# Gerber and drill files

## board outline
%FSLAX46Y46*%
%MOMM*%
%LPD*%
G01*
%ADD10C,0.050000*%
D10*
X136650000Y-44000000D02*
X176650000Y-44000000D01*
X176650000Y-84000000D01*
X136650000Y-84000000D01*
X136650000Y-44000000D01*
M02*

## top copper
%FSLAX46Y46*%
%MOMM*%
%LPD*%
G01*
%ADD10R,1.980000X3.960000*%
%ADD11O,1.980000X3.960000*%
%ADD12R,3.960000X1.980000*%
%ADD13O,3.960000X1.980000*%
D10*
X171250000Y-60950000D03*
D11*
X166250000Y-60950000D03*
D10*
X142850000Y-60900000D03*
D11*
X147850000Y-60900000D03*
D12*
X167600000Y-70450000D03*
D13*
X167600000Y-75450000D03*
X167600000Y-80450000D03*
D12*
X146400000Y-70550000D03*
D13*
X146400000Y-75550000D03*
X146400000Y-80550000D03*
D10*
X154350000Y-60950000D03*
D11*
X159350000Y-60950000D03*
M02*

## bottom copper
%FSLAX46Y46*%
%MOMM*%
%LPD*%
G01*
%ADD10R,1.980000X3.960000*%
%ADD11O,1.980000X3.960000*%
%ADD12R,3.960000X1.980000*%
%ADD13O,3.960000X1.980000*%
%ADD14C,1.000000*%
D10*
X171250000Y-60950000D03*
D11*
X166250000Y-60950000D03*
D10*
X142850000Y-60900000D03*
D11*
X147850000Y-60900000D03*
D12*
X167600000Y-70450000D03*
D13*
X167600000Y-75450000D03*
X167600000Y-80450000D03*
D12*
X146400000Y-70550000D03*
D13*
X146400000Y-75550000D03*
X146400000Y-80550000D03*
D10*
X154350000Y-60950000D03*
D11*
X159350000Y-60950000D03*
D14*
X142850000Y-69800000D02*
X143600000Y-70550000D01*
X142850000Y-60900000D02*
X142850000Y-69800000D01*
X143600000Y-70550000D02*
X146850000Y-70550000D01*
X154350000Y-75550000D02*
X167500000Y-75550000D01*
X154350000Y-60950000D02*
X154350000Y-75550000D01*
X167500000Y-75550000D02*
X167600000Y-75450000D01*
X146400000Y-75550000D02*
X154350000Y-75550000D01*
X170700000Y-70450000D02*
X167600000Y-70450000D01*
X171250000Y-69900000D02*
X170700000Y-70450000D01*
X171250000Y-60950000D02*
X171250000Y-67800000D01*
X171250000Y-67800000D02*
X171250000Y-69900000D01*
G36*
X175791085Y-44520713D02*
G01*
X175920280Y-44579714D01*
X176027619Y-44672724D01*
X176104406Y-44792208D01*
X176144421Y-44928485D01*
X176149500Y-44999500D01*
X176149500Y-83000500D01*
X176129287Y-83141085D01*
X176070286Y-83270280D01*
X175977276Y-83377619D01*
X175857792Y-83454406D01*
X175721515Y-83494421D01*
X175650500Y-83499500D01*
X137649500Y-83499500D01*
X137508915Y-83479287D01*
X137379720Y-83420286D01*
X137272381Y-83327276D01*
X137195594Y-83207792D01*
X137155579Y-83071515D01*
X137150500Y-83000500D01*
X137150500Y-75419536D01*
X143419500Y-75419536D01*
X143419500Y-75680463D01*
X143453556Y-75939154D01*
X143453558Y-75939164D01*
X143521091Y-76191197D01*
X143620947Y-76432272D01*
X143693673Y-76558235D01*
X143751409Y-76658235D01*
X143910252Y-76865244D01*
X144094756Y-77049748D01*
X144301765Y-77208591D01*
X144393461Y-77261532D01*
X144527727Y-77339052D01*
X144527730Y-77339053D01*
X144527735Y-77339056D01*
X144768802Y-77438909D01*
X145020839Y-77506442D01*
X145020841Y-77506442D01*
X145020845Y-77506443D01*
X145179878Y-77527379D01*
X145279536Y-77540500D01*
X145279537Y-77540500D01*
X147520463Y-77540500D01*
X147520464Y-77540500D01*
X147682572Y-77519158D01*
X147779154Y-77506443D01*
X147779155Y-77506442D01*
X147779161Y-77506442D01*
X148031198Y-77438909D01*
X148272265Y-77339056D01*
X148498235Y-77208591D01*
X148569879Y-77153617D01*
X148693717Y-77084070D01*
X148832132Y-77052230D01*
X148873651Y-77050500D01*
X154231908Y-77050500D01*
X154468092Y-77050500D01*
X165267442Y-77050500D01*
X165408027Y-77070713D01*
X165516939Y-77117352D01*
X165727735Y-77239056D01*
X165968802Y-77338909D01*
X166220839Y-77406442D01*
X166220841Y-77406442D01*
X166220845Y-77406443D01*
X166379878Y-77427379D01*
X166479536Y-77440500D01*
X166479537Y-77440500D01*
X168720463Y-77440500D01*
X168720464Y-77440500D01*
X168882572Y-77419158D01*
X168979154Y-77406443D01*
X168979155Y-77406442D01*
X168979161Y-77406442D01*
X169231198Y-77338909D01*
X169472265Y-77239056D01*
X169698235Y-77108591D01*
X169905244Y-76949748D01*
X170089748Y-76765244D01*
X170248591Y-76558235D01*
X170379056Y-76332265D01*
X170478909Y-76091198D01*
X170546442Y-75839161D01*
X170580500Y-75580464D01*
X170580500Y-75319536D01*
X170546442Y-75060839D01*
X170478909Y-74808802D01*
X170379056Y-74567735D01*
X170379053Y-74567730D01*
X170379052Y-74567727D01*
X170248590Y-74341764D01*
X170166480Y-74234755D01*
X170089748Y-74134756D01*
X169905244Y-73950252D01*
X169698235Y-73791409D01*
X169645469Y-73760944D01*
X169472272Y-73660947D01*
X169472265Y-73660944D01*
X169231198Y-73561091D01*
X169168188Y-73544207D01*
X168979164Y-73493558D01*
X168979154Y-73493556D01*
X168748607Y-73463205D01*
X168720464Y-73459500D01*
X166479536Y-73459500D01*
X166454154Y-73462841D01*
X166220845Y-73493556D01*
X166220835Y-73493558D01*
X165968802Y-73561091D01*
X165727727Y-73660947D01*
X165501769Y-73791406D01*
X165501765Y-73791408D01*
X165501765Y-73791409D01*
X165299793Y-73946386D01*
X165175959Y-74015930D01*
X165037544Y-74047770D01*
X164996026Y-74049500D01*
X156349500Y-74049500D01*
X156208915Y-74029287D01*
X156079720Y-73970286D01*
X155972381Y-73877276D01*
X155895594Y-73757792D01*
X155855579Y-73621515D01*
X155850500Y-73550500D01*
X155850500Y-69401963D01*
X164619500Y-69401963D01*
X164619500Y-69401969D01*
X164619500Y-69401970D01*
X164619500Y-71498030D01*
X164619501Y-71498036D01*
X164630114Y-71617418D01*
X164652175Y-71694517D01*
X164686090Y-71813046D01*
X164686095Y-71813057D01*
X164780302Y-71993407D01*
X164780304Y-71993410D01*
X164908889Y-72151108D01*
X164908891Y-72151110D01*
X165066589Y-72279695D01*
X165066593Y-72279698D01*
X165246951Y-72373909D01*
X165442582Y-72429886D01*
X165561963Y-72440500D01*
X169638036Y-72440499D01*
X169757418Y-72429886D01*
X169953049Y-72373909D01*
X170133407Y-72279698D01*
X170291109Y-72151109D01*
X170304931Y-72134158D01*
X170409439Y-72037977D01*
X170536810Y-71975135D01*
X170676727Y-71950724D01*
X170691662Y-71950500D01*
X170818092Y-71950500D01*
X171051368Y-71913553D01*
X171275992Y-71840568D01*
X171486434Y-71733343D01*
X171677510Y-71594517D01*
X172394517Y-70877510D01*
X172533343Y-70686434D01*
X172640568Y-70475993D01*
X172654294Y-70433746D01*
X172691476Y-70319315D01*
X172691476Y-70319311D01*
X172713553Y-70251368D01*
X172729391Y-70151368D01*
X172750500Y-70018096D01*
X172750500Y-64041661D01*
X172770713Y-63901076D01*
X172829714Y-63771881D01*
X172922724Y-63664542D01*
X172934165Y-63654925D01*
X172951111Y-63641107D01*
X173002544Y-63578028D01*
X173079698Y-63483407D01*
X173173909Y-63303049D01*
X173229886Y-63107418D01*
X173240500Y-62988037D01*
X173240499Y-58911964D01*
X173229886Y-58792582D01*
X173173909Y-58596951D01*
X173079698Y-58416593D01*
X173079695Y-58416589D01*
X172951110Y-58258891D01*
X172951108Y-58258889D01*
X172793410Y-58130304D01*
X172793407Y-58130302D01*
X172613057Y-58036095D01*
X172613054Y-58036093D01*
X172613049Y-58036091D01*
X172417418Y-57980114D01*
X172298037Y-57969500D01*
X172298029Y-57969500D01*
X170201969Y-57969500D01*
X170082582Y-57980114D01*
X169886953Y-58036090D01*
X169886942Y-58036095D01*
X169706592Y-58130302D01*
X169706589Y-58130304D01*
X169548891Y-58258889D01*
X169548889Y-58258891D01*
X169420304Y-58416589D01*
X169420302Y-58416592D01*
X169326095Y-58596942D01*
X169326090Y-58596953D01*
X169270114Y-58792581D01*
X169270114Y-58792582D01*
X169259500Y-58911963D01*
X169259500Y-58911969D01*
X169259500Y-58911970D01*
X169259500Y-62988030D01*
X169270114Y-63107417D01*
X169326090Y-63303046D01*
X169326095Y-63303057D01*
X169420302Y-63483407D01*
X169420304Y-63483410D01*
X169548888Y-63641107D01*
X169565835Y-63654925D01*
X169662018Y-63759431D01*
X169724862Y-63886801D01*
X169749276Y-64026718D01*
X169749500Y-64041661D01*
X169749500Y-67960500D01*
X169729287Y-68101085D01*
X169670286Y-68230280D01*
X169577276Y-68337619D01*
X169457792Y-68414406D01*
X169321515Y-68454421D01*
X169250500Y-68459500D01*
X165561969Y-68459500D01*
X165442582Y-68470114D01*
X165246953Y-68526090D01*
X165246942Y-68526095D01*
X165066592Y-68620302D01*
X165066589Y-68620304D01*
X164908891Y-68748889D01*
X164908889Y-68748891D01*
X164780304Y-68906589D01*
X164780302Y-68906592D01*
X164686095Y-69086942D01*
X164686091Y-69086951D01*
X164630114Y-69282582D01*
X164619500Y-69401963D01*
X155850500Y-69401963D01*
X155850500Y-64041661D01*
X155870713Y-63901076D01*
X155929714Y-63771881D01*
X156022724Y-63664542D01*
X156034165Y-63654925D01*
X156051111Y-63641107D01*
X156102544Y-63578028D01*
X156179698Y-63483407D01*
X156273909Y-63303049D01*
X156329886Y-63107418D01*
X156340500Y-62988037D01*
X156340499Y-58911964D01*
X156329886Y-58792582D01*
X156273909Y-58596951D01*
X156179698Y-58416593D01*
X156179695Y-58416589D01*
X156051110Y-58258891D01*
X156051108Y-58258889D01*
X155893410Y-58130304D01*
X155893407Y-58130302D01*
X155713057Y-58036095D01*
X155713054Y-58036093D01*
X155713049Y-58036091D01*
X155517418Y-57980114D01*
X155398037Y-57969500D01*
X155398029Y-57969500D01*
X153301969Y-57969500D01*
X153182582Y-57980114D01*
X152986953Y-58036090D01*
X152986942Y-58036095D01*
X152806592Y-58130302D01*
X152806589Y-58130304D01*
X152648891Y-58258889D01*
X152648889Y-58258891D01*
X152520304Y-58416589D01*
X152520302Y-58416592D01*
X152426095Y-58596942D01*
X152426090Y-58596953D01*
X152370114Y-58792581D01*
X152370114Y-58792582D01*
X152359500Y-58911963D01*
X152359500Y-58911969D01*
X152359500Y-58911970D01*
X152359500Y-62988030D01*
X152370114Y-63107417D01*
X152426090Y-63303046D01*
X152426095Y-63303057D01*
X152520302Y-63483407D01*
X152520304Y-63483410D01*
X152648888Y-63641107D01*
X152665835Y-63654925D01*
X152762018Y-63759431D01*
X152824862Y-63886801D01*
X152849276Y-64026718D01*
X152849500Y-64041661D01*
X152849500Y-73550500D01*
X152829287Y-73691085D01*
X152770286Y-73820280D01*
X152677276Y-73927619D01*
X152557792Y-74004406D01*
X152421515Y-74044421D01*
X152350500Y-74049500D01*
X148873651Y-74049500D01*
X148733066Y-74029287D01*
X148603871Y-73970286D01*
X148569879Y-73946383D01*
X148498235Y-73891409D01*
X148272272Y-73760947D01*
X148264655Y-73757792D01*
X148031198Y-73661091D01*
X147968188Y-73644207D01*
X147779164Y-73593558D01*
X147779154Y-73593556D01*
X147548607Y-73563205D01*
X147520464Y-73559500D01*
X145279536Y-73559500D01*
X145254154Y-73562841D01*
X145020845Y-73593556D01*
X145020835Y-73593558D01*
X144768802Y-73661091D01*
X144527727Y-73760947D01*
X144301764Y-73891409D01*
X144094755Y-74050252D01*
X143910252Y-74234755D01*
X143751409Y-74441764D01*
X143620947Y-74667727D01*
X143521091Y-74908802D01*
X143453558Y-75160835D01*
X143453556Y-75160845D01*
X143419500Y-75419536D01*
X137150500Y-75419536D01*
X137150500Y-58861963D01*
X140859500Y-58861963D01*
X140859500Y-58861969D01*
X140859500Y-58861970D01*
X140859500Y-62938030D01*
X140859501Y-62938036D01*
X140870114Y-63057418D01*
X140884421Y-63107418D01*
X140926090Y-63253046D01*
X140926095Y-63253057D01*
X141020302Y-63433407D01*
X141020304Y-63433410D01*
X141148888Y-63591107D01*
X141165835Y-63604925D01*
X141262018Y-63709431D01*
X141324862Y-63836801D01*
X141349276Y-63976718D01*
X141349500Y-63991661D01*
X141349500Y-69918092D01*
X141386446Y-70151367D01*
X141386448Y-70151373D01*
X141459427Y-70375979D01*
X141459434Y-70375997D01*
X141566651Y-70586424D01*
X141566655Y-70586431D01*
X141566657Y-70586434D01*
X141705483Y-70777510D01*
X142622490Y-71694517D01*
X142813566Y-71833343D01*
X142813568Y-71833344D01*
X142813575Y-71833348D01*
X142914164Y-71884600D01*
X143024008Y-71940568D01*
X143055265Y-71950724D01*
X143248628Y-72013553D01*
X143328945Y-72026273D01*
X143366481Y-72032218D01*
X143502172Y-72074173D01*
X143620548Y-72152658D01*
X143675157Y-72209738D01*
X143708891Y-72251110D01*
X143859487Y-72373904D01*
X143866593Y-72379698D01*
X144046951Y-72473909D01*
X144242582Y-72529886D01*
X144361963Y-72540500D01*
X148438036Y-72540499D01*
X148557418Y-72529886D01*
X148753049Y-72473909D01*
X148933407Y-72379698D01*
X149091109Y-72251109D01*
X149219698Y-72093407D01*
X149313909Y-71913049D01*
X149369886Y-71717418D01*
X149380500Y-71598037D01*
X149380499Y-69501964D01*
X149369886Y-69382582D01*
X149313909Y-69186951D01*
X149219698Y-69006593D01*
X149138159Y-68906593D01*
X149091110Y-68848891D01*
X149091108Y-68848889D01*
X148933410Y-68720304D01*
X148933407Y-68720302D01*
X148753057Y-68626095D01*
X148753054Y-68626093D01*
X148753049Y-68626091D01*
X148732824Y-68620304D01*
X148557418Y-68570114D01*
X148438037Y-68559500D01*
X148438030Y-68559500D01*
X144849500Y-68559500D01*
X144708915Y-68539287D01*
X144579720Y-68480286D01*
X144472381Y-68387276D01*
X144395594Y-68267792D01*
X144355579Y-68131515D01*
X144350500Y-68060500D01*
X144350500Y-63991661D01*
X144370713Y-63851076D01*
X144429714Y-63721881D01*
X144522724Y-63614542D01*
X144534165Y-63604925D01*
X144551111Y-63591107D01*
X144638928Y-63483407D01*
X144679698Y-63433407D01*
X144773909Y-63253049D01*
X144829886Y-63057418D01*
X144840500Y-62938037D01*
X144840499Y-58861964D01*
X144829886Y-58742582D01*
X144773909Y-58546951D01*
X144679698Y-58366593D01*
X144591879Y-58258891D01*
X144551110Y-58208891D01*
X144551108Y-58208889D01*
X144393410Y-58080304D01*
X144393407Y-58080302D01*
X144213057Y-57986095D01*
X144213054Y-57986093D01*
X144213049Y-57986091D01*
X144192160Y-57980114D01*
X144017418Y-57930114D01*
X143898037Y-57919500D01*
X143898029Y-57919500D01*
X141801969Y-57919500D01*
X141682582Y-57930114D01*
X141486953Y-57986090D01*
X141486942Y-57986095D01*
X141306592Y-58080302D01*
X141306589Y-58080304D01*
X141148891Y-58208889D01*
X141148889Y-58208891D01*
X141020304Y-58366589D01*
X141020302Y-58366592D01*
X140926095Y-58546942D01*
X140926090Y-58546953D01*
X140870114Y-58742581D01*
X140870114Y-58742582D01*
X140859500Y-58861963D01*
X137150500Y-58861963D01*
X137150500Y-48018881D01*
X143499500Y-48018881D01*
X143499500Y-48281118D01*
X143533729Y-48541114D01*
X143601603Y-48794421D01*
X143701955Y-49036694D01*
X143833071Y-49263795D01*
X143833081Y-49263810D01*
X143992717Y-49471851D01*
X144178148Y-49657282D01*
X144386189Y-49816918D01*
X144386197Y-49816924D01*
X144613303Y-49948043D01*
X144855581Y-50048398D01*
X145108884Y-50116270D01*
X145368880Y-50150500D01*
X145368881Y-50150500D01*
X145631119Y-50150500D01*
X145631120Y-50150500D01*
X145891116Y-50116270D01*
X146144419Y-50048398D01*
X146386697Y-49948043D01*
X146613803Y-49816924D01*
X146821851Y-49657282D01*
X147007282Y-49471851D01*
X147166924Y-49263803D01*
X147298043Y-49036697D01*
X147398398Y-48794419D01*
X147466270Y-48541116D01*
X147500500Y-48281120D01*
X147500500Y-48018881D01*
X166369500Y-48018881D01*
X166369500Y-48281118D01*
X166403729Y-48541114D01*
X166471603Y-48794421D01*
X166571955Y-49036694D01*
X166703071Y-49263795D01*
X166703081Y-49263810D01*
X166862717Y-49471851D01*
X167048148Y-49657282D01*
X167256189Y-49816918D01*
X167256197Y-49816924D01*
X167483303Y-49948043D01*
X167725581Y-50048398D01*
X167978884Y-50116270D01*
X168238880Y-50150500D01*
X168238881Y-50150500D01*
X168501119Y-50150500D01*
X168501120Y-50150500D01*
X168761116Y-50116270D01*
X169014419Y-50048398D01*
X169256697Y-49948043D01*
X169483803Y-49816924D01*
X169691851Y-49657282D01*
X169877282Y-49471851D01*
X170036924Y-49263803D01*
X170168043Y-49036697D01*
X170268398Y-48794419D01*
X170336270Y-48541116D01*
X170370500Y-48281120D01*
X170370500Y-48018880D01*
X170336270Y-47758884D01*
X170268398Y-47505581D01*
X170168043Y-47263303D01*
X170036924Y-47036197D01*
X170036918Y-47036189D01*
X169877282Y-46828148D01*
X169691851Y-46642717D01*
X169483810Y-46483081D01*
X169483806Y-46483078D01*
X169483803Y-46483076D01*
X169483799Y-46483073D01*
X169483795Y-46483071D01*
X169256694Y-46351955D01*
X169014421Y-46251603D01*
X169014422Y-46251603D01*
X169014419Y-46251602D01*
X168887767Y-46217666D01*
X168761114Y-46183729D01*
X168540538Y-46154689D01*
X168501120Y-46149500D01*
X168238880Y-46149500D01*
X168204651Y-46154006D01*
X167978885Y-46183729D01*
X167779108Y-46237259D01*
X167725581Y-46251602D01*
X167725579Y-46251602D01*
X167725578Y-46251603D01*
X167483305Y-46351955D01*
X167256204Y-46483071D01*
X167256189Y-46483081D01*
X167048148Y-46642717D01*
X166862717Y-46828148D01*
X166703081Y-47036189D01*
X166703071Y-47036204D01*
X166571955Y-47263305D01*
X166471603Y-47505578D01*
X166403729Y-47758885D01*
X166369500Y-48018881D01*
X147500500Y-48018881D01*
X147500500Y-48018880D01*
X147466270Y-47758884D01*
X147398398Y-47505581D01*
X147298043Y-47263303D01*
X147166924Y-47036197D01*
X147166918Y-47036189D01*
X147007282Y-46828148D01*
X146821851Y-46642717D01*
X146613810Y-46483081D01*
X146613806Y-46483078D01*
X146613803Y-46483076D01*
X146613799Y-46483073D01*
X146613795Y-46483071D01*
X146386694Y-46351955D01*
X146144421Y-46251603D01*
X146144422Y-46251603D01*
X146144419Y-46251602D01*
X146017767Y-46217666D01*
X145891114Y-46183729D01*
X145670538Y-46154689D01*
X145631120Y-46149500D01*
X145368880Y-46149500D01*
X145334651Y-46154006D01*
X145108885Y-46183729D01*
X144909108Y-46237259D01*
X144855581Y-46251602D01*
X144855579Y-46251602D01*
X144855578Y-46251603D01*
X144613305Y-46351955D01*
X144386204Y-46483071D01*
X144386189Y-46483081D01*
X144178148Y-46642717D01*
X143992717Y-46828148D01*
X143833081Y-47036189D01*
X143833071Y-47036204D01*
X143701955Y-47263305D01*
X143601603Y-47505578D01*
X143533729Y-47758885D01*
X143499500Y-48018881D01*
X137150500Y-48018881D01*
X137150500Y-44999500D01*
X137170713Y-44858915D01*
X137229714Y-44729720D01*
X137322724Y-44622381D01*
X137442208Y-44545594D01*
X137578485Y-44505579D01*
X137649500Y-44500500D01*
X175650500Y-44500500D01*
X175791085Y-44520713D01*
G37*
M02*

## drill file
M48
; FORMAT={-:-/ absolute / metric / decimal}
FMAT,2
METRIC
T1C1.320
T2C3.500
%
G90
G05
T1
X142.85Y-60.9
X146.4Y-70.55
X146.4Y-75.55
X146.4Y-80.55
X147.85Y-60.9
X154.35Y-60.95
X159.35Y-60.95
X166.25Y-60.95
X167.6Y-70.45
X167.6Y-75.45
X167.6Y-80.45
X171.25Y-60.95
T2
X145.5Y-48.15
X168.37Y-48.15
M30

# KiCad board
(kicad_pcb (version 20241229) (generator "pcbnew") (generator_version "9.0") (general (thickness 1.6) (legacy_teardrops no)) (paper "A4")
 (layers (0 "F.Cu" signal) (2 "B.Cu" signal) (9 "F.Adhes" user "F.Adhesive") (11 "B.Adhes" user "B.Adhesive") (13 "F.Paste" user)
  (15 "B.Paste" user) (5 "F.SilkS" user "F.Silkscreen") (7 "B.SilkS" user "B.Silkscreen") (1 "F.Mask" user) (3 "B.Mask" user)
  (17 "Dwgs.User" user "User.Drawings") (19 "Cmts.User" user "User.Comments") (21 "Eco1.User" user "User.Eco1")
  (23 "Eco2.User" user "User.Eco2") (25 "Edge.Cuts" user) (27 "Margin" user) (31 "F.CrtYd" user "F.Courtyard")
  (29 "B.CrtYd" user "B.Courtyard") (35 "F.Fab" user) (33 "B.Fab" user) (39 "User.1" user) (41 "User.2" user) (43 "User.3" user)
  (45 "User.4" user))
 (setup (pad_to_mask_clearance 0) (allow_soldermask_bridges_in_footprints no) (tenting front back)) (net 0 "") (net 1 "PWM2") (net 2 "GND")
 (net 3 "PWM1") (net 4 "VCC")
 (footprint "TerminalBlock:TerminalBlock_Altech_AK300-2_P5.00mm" (layer "F.Cu") (at 171.25 60.95 180)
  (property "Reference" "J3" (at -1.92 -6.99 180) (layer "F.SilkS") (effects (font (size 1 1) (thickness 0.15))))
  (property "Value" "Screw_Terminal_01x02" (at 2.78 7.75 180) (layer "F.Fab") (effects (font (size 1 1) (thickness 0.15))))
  (pad "1" thru_hole rect (at 0 0 180) (size 1.98 3.96) (drill 1.32) (layers "*.Cu" "*.Mask") (remove_unused_layers no) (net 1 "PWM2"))
  (pad "2" thru_hole oval (at 5 0 180) (size 1.98 3.96) (drill 1.32) (layers "*.Cu" "*.Mask") (remove_unused_layers no) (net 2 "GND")))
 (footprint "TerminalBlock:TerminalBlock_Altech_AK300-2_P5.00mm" (layer "F.Cu") (at 142.85 60.9)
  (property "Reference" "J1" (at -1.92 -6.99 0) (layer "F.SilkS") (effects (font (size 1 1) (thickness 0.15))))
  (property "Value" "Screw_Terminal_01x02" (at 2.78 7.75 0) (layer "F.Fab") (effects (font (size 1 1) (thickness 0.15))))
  (pad "1" thru_hole rect (at 0 0) (size 1.98 3.96) (drill 1.32) (layers "*.Cu" "*.Mask") (remove_unused_layers no) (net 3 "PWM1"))
  (pad "2" thru_hole oval (at 5 0) (size 1.98 3.96) (drill 1.32) (layers "*.Cu" "*.Mask") (remove_unused_layers no) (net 2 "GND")))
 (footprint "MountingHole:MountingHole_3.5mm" (layer "F.Cu") (at 168.37 48.15)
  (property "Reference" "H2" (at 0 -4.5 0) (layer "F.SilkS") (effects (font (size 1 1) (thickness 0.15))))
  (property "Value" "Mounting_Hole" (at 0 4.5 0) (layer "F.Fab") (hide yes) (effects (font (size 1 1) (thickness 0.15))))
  (pad "" np_thru_hole circle (at 0 0) (size 3.5 3.5) (drill 3.5) (layers "*.Cu" "*.Mask")))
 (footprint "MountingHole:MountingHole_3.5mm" (layer "F.Cu") (at 145.5 48.15)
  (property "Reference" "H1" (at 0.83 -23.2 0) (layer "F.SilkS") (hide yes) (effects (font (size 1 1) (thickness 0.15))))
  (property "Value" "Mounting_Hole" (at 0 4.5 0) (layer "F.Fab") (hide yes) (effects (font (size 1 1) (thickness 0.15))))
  (pad "" np_thru_hole circle (at 0 0) (size 3.5 3.5) (drill 3.5) (layers "*.Cu" "*.Mask")))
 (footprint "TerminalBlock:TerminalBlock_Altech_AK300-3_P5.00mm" (layer "F.Cu") (at 167.6 70.45 -90)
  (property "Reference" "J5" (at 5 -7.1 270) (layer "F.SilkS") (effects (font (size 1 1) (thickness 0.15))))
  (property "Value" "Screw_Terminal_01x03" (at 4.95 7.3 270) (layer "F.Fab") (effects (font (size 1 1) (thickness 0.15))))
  (pad "1" thru_hole rect (at 0 0 270) (size 1.98 3.96) (drill 1.32) (layers "*.Cu" "*.Mask") (remove_unused_layers no) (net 1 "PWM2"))
  (pad "2" thru_hole oval (at 5 0 270) (size 1.98 3.96) (drill 1.32) (layers "*.Cu" "*.Mask") (remove_unused_layers no) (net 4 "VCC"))
  (pad "3" thru_hole oval (at 10 0 270) (size 1.98 3.96) (drill 1.32) (layers "*.Cu" "*.Mask") (remove_unused_layers no) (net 2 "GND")))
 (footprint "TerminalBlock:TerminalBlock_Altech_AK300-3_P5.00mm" (layer "F.Cu") (at 146.4 70.55 -90)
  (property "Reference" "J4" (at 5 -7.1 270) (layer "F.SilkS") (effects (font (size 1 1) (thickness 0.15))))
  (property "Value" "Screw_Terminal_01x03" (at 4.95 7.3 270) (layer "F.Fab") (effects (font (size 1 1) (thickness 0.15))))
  (pad "1" thru_hole rect (at 0 0 270) (size 1.98 3.96) (drill 1.32) (layers "*.Cu" "*.Mask") (remove_unused_layers no) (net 3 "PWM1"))
  (pad "2" thru_hole oval (at 5 0 270) (size 1.98 3.96) (drill 1.32) (layers "*.Cu" "*.Mask") (remove_unused_layers no) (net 4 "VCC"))
  (pad "3" thru_hole oval (at 10 0 270) (size 1.98 3.96) (drill 1.32) (layers "*.Cu" "*.Mask") (remove_unused_layers no) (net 2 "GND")))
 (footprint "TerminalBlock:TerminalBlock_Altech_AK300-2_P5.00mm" (layer "F.Cu") (at 154.35 60.95)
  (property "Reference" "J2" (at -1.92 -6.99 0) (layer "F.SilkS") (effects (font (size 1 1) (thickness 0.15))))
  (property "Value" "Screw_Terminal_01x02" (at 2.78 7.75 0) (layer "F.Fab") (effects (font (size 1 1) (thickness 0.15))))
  (pad "1" thru_hole rect (at 0 0) (size 1.98 3.96) (drill 1.32) (layers "*.Cu" "*.Mask") (remove_unused_layers no) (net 4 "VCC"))
  (pad "2" thru_hole oval (at 5 0) (size 1.98 3.96) (drill 1.32) (layers "*.Cu" "*.Mask") (remove_unused_layers no) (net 2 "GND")))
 (gr_rect (start 136.65 44) (end 176.65 84) (stroke (width 0.05) (type default)) (fill no) (layer "Edge.Cuts"))
 (segment (start 142.85 69.8) (end 143.6 70.55) (width 1) (layer "B.Cu") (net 3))
 (segment (start 142.85 60.9) (end 142.85 69.8) (width 1) (layer "B.Cu") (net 3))
 (segment (start 143.6 70.55) (end 146.85 70.55) (width 1) (layer "B.Cu") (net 3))
 (segment (start 154.35 75.55) (end 167.5 75.55) (width 1) (layer "B.Cu") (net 4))
 (segment (start 154.35 60.95) (end 154.35 75.55) (width 1) (layer "B.Cu") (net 4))
 (segment (start 167.5 75.55) (end 167.6 75.45) (width 1) (layer "B.Cu") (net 4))
 (segment (start 146.4 75.55) (end 154.35 75.55) (width 1) (layer "B.Cu") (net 4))
 (segment (start 170.7 70.45) (end 167.6 70.45) (width 1) (layer "B.Cu") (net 1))
 (segment (start 171.25 69.9) (end 170.7 70.45) (width 1) (layer "B.Cu") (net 1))
 (segment (start 171.25 60.95) (end 171.25 67.8) (width 1) (layer "B.Cu") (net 1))
 (segment (start 171.25 67.8) (end 171.25 69.9) (width 1) (layer "B.Cu") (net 1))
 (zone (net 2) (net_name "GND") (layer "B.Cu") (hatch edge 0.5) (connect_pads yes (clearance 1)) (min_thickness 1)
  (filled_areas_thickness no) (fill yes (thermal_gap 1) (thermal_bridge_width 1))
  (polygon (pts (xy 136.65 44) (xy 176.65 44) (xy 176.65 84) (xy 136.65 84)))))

